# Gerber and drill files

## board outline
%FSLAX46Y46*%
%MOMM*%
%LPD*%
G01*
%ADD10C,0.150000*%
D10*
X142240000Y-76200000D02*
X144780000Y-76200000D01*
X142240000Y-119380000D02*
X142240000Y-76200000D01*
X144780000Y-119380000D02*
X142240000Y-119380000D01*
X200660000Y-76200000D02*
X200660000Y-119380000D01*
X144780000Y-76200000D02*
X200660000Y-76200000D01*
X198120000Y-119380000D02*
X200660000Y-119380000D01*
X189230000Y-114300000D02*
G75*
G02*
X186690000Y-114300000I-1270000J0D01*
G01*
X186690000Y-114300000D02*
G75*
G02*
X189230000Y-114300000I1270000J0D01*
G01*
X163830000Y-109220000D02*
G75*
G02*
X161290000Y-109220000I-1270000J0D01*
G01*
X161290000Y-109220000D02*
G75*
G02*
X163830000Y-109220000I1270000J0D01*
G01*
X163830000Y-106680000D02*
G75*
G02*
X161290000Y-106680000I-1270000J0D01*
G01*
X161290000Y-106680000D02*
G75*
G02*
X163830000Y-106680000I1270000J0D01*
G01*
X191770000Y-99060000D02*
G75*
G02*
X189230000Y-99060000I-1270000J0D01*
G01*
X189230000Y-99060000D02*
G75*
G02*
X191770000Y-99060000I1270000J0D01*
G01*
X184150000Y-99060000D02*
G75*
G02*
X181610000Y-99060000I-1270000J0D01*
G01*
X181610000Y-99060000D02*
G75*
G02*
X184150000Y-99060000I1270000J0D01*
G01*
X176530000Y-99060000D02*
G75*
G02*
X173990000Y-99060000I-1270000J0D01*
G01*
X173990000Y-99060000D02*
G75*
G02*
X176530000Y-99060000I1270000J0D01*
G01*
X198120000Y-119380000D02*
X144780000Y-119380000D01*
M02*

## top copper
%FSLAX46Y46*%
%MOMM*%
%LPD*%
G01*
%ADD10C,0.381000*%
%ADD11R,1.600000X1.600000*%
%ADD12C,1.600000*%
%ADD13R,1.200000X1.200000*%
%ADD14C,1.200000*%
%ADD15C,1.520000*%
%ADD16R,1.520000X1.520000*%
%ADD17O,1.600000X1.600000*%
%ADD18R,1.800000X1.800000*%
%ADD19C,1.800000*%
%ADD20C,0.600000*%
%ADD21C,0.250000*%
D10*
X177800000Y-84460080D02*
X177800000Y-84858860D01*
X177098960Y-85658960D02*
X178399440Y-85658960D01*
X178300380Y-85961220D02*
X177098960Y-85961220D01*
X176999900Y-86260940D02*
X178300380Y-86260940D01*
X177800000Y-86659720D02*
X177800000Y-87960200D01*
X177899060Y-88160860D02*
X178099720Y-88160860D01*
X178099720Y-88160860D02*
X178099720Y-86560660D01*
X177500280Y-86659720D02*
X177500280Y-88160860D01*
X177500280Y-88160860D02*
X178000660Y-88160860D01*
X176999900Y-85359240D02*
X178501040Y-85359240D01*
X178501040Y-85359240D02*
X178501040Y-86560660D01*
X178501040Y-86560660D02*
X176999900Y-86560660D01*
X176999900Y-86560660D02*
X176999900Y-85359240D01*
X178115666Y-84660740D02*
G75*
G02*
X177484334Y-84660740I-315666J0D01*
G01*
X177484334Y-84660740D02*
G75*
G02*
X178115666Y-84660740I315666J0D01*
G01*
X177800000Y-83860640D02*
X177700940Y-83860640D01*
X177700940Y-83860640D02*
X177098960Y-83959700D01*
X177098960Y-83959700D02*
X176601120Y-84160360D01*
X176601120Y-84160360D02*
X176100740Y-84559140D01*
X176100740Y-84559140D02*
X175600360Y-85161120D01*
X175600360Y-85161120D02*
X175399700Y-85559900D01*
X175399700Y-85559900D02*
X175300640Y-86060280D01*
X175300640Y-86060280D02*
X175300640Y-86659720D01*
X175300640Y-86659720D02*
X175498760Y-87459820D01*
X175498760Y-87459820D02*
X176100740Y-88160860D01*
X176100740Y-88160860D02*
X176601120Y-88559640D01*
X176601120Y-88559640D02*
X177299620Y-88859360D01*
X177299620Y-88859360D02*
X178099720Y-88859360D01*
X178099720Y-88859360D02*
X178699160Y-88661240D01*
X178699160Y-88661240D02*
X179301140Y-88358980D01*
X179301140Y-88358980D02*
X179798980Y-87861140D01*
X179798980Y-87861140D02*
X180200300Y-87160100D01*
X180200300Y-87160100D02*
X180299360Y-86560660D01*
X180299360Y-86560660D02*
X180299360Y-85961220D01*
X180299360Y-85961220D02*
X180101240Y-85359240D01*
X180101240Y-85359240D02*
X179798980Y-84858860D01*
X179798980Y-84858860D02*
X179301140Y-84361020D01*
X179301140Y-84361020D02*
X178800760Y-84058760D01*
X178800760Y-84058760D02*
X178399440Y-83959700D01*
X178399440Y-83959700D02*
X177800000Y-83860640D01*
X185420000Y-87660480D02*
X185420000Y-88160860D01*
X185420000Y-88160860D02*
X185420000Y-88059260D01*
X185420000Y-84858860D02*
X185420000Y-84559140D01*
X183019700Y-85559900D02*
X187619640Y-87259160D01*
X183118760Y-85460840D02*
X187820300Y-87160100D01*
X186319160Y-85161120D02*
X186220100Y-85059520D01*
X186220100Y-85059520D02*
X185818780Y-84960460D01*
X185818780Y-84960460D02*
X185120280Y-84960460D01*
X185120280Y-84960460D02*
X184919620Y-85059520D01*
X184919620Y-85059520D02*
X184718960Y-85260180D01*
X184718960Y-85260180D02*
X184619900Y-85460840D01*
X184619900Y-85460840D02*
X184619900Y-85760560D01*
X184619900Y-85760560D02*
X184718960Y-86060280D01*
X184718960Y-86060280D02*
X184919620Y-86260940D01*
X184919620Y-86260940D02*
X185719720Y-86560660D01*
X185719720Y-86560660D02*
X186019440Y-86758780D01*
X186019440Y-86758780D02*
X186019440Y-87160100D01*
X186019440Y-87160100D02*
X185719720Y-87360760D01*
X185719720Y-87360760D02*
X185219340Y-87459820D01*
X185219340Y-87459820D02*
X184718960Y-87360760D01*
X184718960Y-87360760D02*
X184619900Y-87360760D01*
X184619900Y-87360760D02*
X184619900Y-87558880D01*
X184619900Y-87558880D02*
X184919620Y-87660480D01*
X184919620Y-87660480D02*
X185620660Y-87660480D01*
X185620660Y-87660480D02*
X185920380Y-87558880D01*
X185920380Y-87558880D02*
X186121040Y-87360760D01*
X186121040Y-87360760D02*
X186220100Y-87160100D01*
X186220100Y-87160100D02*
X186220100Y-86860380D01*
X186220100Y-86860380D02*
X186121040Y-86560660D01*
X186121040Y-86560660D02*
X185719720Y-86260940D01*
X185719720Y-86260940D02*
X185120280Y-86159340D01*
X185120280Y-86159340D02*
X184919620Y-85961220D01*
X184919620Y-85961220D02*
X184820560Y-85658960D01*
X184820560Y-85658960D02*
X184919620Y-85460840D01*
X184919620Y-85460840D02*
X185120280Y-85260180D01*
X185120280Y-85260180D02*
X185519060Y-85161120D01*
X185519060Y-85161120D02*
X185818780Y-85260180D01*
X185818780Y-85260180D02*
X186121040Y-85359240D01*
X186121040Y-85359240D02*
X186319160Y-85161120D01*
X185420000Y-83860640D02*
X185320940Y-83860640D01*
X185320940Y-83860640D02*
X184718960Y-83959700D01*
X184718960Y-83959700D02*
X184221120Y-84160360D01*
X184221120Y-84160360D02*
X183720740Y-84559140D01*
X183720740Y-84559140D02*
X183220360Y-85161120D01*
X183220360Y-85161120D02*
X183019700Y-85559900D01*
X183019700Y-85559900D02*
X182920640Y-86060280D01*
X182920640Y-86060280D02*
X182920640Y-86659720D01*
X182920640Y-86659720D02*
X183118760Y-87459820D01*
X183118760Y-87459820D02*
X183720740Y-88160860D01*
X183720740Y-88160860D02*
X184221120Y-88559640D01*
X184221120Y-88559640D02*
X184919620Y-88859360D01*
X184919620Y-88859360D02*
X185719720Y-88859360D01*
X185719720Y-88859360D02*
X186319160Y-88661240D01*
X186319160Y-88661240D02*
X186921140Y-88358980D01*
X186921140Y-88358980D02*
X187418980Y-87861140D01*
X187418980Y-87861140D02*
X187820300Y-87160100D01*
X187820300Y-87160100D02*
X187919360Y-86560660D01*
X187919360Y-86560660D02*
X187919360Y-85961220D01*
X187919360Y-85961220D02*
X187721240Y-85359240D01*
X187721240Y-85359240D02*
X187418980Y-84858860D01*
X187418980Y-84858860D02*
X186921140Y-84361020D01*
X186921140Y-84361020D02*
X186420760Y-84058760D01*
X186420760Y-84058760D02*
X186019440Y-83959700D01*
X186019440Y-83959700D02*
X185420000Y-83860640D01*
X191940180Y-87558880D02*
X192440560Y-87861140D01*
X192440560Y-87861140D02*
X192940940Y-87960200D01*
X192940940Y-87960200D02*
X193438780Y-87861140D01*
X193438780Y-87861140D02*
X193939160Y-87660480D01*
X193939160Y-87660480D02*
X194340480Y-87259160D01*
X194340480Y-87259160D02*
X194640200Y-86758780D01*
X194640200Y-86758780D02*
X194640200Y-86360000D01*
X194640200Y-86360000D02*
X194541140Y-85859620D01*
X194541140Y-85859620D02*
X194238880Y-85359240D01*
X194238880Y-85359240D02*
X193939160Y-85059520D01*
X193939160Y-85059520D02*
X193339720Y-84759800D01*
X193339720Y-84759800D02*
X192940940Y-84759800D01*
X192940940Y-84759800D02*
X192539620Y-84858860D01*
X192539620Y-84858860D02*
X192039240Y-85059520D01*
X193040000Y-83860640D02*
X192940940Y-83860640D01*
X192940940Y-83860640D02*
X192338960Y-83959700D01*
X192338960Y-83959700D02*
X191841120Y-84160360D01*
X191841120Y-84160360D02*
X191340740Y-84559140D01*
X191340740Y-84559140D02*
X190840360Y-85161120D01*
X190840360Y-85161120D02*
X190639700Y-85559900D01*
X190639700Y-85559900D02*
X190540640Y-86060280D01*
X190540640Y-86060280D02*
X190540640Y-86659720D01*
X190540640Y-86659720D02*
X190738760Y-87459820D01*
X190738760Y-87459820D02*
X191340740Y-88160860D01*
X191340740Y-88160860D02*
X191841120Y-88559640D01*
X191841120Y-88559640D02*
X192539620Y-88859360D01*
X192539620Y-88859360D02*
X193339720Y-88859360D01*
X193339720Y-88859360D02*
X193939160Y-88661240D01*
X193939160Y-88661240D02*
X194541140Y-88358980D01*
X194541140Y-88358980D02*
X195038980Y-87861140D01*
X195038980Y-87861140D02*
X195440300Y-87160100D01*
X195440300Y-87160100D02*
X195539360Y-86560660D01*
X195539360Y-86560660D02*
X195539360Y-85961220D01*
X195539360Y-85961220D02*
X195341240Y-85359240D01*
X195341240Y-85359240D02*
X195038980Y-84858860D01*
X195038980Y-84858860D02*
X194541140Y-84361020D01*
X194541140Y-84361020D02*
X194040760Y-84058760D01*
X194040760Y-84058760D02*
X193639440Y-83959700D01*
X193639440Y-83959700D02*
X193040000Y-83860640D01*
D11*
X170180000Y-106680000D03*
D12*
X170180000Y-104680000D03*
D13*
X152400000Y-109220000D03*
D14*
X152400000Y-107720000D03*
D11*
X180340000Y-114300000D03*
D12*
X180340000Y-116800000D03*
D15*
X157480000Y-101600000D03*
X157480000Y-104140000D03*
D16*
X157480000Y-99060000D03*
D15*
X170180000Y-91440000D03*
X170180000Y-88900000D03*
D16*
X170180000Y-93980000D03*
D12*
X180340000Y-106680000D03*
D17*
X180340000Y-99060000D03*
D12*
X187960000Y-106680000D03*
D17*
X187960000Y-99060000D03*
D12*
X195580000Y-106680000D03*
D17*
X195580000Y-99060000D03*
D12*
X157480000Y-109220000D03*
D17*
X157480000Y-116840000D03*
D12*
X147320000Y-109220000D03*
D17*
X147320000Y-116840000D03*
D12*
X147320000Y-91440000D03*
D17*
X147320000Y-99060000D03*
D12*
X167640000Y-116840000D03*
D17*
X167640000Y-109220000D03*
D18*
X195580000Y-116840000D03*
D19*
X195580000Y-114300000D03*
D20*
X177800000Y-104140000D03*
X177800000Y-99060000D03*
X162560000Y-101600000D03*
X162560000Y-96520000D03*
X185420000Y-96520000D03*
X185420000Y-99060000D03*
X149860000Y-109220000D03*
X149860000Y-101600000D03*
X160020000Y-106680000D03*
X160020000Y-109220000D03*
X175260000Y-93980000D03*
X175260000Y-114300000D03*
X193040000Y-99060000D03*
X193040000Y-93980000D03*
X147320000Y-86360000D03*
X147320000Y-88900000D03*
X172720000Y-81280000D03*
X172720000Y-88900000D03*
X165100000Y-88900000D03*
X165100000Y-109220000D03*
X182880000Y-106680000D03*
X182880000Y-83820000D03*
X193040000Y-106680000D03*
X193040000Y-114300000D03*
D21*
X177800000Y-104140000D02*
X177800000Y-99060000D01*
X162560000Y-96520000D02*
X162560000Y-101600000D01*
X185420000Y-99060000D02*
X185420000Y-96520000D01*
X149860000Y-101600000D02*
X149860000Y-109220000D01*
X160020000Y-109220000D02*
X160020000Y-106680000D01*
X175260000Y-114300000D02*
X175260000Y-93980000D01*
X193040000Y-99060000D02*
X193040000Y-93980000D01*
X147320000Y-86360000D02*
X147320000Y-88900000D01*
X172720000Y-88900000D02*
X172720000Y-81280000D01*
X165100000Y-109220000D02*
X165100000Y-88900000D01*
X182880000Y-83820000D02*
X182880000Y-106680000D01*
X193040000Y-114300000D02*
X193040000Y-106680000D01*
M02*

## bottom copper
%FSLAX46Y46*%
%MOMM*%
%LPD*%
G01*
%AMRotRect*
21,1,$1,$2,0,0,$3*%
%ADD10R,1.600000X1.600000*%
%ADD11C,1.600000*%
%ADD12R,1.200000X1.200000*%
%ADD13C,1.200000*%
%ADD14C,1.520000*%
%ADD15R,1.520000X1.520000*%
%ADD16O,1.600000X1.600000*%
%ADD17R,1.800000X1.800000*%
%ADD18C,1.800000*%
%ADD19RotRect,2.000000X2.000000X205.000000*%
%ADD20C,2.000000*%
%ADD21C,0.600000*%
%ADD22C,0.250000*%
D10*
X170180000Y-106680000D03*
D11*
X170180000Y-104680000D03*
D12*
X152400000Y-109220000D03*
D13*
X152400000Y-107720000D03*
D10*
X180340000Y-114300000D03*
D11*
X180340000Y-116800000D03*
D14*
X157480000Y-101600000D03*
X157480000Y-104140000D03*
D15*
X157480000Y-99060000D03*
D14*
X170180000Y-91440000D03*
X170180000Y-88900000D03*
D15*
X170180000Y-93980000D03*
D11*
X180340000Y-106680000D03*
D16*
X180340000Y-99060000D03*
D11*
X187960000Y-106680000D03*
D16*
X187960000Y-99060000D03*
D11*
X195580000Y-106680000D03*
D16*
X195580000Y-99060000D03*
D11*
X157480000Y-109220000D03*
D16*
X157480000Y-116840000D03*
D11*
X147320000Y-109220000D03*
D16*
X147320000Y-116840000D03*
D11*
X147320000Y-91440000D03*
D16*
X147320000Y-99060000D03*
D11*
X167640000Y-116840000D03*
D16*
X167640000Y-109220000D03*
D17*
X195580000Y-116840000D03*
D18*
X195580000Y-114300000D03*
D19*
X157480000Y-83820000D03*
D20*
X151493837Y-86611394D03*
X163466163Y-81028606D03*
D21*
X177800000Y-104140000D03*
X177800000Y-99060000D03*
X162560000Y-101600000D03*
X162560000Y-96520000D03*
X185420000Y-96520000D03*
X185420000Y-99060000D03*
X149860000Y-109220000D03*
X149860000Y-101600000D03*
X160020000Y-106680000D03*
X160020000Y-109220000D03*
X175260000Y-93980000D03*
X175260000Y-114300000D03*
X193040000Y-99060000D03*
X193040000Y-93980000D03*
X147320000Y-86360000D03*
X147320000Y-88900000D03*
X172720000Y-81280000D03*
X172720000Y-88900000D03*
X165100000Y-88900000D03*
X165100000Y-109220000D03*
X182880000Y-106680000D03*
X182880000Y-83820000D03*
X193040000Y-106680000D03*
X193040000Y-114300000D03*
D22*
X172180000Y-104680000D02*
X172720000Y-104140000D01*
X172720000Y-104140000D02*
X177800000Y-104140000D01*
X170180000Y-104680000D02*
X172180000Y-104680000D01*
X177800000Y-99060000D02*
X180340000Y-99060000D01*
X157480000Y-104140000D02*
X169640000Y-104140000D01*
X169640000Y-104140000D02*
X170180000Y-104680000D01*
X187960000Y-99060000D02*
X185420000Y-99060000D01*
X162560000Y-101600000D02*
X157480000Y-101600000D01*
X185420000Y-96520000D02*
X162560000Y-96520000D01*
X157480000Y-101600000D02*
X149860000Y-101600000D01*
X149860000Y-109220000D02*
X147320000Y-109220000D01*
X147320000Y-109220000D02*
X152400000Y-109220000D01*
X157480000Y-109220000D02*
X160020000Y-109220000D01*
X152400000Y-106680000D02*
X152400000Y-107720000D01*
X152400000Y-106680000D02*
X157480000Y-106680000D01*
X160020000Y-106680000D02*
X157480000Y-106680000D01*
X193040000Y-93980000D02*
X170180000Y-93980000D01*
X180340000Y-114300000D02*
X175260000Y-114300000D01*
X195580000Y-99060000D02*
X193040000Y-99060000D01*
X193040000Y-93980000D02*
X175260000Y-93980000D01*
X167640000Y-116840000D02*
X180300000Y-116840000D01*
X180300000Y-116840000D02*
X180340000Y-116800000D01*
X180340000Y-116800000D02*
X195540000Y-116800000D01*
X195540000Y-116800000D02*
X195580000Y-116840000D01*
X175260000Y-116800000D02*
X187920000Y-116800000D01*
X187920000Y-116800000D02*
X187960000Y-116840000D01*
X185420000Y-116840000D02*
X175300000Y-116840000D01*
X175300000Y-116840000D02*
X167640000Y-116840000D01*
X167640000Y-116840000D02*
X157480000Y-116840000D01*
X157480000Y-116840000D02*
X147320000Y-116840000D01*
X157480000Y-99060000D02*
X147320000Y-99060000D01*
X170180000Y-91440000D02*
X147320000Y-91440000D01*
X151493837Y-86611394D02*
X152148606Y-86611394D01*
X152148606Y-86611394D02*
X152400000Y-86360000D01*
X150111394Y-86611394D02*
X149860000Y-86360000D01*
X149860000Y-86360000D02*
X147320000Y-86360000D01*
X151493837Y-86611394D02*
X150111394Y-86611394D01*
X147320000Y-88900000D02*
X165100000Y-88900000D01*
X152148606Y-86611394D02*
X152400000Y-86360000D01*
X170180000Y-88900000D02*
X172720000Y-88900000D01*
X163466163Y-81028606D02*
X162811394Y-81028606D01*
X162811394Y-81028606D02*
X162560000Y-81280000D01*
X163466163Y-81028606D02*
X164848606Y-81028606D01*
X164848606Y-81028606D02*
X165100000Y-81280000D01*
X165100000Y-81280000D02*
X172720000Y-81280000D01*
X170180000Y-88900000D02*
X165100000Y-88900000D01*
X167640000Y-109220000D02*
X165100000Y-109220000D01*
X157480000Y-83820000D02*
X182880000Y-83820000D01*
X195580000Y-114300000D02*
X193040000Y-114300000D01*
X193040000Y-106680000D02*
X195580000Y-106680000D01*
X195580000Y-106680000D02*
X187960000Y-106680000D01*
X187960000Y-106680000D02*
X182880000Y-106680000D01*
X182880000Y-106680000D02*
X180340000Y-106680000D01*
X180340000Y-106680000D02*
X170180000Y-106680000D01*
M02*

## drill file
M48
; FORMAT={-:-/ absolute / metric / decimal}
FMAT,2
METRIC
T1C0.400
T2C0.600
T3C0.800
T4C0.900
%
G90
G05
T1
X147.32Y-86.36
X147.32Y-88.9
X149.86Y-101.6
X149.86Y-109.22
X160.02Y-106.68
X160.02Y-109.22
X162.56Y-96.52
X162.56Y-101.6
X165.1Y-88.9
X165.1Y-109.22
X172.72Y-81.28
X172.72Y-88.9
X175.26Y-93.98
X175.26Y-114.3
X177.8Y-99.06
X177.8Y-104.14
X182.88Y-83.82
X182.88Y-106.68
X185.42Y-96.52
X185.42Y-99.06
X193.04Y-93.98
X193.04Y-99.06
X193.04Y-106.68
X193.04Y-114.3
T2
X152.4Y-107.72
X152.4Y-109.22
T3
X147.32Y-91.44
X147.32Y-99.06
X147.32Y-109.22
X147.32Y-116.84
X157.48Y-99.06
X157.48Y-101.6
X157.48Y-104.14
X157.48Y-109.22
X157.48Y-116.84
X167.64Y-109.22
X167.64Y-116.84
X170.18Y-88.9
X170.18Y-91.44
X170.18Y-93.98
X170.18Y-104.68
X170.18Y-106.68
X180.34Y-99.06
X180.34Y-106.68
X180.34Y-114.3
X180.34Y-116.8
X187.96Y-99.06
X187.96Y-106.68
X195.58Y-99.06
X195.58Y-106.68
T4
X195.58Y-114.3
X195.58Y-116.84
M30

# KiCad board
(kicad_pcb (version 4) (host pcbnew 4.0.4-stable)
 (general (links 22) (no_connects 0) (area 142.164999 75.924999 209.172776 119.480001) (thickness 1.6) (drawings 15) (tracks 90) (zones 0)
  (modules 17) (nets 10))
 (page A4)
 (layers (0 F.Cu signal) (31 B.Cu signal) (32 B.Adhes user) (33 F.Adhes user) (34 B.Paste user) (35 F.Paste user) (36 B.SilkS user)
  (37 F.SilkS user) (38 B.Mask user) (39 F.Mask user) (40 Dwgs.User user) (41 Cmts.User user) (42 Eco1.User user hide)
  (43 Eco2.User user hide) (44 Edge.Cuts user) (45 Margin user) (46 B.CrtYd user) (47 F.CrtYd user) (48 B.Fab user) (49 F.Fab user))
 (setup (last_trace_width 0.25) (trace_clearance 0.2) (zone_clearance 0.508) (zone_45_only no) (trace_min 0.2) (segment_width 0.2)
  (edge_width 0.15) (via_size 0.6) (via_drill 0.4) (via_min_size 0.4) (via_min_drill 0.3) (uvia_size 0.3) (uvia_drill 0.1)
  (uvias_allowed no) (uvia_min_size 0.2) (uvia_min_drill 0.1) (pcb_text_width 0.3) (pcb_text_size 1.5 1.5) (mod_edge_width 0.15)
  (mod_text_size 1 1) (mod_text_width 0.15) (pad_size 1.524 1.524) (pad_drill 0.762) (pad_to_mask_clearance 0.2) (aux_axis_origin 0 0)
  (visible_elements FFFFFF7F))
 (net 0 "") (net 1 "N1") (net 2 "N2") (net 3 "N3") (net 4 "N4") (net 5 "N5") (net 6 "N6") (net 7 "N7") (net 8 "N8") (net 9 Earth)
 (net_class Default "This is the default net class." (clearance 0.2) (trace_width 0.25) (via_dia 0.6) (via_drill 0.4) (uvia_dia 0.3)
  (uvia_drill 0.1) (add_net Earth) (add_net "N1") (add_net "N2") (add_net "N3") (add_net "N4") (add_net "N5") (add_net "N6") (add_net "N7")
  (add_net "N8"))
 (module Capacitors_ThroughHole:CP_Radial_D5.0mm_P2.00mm (layer F.Cu) (at 170.18 106.68 90)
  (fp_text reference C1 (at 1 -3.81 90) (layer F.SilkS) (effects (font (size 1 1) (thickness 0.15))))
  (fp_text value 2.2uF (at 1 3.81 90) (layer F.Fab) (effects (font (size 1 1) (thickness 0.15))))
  (pad 1 thru_hole rect (at 0 0 90) (size 1.6 1.6) (drill 0.8) (layers *.Cu *.Mask) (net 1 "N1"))
  (pad 2 thru_hole circle (at 2 0 90) (size 1.6 1.6) (drill 0.8) (layers *.Cu *.Mask) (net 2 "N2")))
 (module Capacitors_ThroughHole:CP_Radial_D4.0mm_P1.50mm (layer F.Cu) (at 152.4 109.22 90)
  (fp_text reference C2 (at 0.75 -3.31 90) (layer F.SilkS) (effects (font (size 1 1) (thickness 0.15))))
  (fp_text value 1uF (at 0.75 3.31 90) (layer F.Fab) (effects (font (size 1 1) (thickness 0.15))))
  (pad 1 thru_hole rect (at 0 0 90) (size 1.2 1.2) (drill 0.6) (layers *.Cu *.Mask) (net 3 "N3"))
  (pad 2 thru_hole circle (at 1.5 0 90) (size 1.2 1.2) (drill 0.6) (layers *.Cu *.Mask) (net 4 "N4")))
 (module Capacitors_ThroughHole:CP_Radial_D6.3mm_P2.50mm (layer F.Cu) (at 180.34 114.3 270)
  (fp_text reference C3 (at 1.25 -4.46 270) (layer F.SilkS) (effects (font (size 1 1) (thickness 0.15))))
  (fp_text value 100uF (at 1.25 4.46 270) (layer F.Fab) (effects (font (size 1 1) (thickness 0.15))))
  (pad 1 thru_hole rect (at 0 0 270) (size 1.6 1.6) (drill 0.8) (layers *.Cu *.Mask) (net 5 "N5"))
  (pad 2 thru_hole circle (at 2.5 0 270) (size 1.6 1.6) (drill 0.8) (layers *.Cu *.Mask) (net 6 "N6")))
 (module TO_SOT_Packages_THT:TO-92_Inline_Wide (layer F.Cu) (at 157.48 99.06 270)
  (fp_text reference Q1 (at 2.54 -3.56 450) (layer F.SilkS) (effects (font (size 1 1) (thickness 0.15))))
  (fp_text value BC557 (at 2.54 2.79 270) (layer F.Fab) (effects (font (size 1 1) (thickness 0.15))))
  (pad 2 thru_hole circle (at 2.54 0) (size 1.52 1.52) (drill 0.8) (layers *.Cu *.Mask) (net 3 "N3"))
  (pad 3 thru_hole circle (at 5.08 0) (size 1.52 1.52) (drill 0.8) (layers *.Cu *.Mask) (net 2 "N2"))
  (pad 1 thru_hole rect (at 0 0) (size 1.52 1.52) (drill 0.8) (layers *.Cu *.Mask) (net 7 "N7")))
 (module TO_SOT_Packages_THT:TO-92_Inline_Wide (layer F.Cu) (at 170.18 93.98 90)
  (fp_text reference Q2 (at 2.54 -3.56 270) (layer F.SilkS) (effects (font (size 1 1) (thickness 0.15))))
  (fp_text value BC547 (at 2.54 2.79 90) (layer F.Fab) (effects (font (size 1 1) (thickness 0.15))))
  (pad 2 thru_hole circle (at 2.54 0 180) (size 1.52 1.52) (drill 0.8) (layers *.Cu *.Mask) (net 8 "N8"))
  (pad 3 thru_hole circle (at 5.08 0 180) (size 1.52 1.52) (drill 0.8) (layers *.Cu *.Mask) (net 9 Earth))
  (pad 1 thru_hole rect (at 0 0 180) (size 1.52 1.52) (drill 0.8) (layers *.Cu *.Mask) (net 5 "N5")))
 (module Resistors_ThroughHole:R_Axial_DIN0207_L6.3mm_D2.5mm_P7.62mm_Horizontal (layer F.Cu) (at 180.34 106.68 90)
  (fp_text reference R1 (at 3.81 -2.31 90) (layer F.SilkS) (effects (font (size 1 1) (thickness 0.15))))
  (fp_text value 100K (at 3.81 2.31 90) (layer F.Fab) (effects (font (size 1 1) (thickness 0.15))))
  (pad 1 thru_hole circle (at 0 0 90) (size 1.6 1.6) (drill 0.8) (layers *.Cu *.Mask) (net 1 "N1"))
  (pad 2 thru_hole oval (at 7.62 0 90) (size 1.6 1.6) (drill 0.8) (layers *.Cu *.Mask) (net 2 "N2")))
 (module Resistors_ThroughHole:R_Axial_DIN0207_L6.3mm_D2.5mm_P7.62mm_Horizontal (layer F.Cu) (at 187.96 106.68 90)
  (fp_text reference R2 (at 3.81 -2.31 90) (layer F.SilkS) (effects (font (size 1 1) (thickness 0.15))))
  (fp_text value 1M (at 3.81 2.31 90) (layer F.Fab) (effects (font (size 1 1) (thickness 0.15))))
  (pad 1 thru_hole circle (at 0 0 90) (size 1.6 1.6) (drill 0.8) (layers *.Cu *.Mask) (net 1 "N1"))
  (pad 2 thru_hole oval (at 7.62 0 90) (size 1.6 1.6) (drill 0.8) (layers *.Cu *.Mask) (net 3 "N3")))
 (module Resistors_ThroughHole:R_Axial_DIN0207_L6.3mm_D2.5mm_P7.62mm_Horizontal (layer F.Cu) (at 195.58 106.68 90)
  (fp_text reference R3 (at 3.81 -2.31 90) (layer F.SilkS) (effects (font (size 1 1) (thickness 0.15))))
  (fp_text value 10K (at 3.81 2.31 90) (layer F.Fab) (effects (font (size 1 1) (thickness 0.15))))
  (pad 1 thru_hole circle (at 0 0 90) (size 1.6 1.6) (drill 0.8) (layers *.Cu *.Mask) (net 1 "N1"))
  (pad 2 thru_hole oval (at 7.62 0 90) (size 1.6 1.6) (drill 0.8) (layers *.Cu *.Mask) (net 5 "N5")))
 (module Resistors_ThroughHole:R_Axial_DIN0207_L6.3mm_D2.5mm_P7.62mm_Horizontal (layer F.Cu) (at 157.48 109.22 270)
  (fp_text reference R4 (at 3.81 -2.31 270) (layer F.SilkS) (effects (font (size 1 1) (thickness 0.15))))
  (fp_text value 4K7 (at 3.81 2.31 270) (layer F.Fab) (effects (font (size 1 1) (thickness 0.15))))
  (pad 1 thru_hole circle (at 0 0 270) (size 1.6 1.6) (drill 0.8) (layers *.Cu *.Mask) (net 4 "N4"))
  (pad 2 thru_hole oval (at 7.62 0 270) (size 1.6 1.6) (drill 0.8) (layers *.Cu *.Mask) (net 6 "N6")))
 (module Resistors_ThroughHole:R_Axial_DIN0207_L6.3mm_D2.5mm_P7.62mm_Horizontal (layer F.Cu) (at 147.32 109.22 270)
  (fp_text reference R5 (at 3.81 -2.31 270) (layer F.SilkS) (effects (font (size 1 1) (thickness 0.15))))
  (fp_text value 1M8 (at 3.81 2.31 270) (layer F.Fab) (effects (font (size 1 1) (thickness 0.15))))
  (pad 1 thru_hole circle (at 0 0 270) (size 1.6 1.6) (drill 0.8) (layers *.Cu *.Mask) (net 3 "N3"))
  (pad 2 thru_hole oval (at 7.62 0 270) (size 1.6 1.6) (drill 0.8) (layers *.Cu *.Mask) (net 6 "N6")))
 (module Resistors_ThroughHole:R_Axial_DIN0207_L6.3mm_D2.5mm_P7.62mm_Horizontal (layer F.Cu) (at 147.32 91.44 270)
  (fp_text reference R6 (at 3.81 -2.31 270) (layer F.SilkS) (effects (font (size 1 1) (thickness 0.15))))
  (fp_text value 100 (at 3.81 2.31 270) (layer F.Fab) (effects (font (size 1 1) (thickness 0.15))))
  (pad 1 thru_hole circle (at 0 0 270) (size 1.6 1.6) (drill 0.8) (layers *.Cu *.Mask) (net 8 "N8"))
  (pad 2 thru_hole oval (at 7.62 0 270) (size 1.6 1.6) (drill 0.8) (layers *.Cu *.Mask) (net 7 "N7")))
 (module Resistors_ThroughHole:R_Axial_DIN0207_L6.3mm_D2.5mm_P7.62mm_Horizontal (layer F.Cu) (at 167.64 116.84 90)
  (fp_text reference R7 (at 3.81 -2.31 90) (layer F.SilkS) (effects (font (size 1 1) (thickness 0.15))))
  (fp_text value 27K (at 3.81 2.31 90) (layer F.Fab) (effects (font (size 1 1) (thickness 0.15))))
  (pad 1 thru_hole circle (at 0 0 90) (size 1.6 1.6) (drill 0.8) (layers *.Cu *.Mask) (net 6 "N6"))
  (pad 2 thru_hole oval (at 7.62 0 90) (size 1.6 1.6) (drill 0.8) (layers *.Cu *.Mask) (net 9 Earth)))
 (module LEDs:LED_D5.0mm (layer F.Cu) (at 195.58 116.84 90)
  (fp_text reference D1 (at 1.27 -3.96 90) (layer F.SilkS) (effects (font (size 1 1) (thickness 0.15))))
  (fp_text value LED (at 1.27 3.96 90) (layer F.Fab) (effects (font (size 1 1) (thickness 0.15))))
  (pad 1 thru_hole rect (at 0 0 90) (size 1.8 1.8) (drill 0.9) (layers *.Cu *.Mask) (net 6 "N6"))
  (pad 2 thru_hole circle (at 2.54 0 90) (size 1.8 1.8) (drill 0.9) (layers *.Cu *.Mask) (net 1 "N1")))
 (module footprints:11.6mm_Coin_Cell (layer F.Cu) (at 157.48 83.82 205) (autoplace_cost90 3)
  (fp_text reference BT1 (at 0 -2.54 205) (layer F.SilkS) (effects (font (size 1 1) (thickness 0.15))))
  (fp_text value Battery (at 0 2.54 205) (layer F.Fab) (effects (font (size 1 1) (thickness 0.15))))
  (pad 1 smd rect (at 0 0 205) (size 2 2) (layers B.Cu F.Paste F.Mask) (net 1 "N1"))
  (pad 2 smd circle (at 6.605 0 205) (size 2 2) (layers B.Cu F.Paste F.Mask) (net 9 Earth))
  (pad 2 smd circle (at -6.605 0 205) (size 2 2) (layers B.Cu F.Paste F.Mask) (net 9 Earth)))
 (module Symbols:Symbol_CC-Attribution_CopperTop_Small (layer F.Cu) (at 177.8 86.36)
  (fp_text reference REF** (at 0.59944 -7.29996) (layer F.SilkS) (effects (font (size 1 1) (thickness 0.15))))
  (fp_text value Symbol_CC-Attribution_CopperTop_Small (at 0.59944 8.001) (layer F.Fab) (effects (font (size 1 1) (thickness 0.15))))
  (fp_line (start 0 -1.89992) (end 0 -1.50114) (layer F.Cu) (width 0.381))
  (fp_line (start -0.70104 -0.70104) (end 0.59944 -0.70104) (layer F.Cu) (width 0.381))
  (fp_line (start 0.50038 -0.39878) (end -0.70104 -0.39878) (layer F.Cu) (width 0.381))
  (fp_line (start -0.8001 -0.09906) (end 0.50038 -0.09906) (layer F.Cu) (width 0.381))
  (fp_line (start 0 0.29972) (end 0 1.6002) (layer F.Cu) (width 0.381))
  (fp_line (start 0.09906 1.80086) (end 0.29972 1.80086) (layer F.Cu) (width 0.381))
  (fp_line (start 0.29972 1.80086) (end 0.29972 0.20066) (layer F.Cu) (width 0.381))
  (fp_line (start -0.29972 0.29972) (end -0.29972 1.80086) (layer F.Cu) (width 0.381))
  (fp_line (start -0.29972 1.80086) (end 0.20066 1.80086) (layer F.Cu) (width 0.381))
  (fp_line (start -0.8001 -1.00076) (end 0.70104 -1.00076) (layer F.Cu) (width 0.381))
  (fp_line (start 0.70104 -1.00076) (end 0.70104 0.20066) (layer F.Cu) (width 0.381))
  (fp_line (start 0.70104 0.20066) (end -0.8001 0.20066) (layer F.Cu) (width 0.381))
  (fp_line (start -0.8001 0.20066) (end -0.8001 -1.00076) (layer F.Cu) (width 0.381))
  (fp_circle (center 0 -1.69926) (end 0.09906 -1.39954) (layer F.Cu) (width 0.381))
  (fp_line (start 0 -2.49936) (end -0.09906 -2.49936) (layer F.Cu) (width 0.381))
  (fp_line (start -0.09906 -2.49936) (end -0.70104 -2.4003) (layer F.Cu) (width 0.381))
  (fp_line (start -0.70104 -2.4003) (end -1.19888 -2.19964) (layer F.Cu) (width 0.381))
  (fp_line (start -1.19888 -2.19964) (end -1.69926 -1.80086) (layer F.Cu) (width 0.381))
  (fp_line (start -1.69926 -1.80086) (end -2.19964 -1.19888) (layer F.Cu) (width 0.381))
  (fp_line (start -2.19964 -1.19888) (end -2.4003 -0.8001) (layer F.Cu) (width 0.381))
  (fp_line (start -2.4003 -0.8001) (end -2.49936 -0.29972) (layer F.Cu) (width 0.381))
  (fp_line (start -2.49936 -0.29972) (end -2.49936 0.29972) (layer F.Cu) (width 0.381))
  (fp_line (start -2.49936 0.29972) (end -2.30124 1.09982) (layer F.Cu) (width 0.381))
  (fp_line (start -2.30124 1.09982) (end -1.69926 1.80086) (layer F.Cu) (width 0.381))
  (fp_line (start -1.69926 1.80086) (end -1.19888 2.19964) (layer F.Cu) (width 0.381))
  (fp_line (start -1.19888 2.19964) (end -0.50038 2.49936) (layer F.Cu) (width 0.381))
  (fp_line (start -0.50038 2.49936) (end 0.29972 2.49936) (layer F.Cu) (width 0.381))
  (fp_line (start 0.29972 2.49936) (end 0.89916 2.30124) (layer F.Cu) (width 0.381))
  (fp_line (start 0.89916 2.30124) (end 1.50114 1.99898) (layer F.Cu) (width 0.381))
  (fp_line (start 1.50114 1.99898) (end 1.99898 1.50114) (layer F.Cu) (width 0.381))
  (fp_line (start 1.99898 1.50114) (end 2.4003 0.8001) (layer F.Cu) (width 0.381))
  (fp_line (start 2.4003 0.8001) (end 2.49936 0.20066) (layer F.Cu) (width 0.381))
  (fp_line (start 2.49936 0.20066) (end 2.49936 -0.39878) (layer F.Cu) (width 0.381))
  (fp_line (start 2.49936 -0.39878) (end 2.30124 -1.00076) (layer F.Cu) (width 0.381))
  (fp_line (start 2.30124 -1.00076) (end 1.99898 -1.50114) (layer F.Cu) (width 0.381))
  (fp_line (start 1.99898 -1.50114) (end 1.50114 -1.99898) (layer F.Cu) (width 0.381))
  (fp_line (start 1.50114 -1.99898) (end 1.00076 -2.30124) (layer F.Cu) (width 0.381))
  (fp_line (start 1.00076 -2.30124) (end 0.59944 -2.4003) (layer F.Cu) (width 0.381))
  (fp_line (start 0.59944 -2.4003) (end 0 -2.49936) (layer F.Cu) (width 0.381)))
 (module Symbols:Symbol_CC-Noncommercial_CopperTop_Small (layer F.Cu) (at 185.42 86.36)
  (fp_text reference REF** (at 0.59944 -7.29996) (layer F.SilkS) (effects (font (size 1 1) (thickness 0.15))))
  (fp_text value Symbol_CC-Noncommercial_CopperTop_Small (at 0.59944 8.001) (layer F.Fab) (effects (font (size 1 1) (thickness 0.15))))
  (fp_line (start 0 1.30048) (end 0 1.80086) (layer F.Cu) (width 0.381))
  (fp_line (start 0 1.80086) (end 0 1.69926) (layer F.Cu) (width 0.381))
  (fp_line (start 0 -1.50114) (end 0 -1.80086) (layer F.Cu) (width 0.381))
  (fp_line (start -2.4003 -0.8001) (end 2.19964 0.89916) (layer F.Cu) (width 0.381))
  (fp_line (start -2.30124 -0.89916) (end 2.4003 0.8001) (layer F.Cu) (width 0.381))
  (fp_line (start 0.89916 -1.19888) (end 0.8001 -1.30048) (layer F.Cu) (width 0.381))
  (fp_line (start 0.8001 -1.30048) (end 0.39878 -1.39954) (layer F.Cu) (width 0.381))
  (fp_line (start 0.39878 -1.39954) (end -0.29972 -1.39954) (layer F.Cu) (width 0.381))
  (fp_line (start -0.29972 -1.39954) (end -0.50038 -1.30048) (layer F.Cu) (width 0.381))
  (fp_line (start -0.50038 -1.30048) (end -0.70104 -1.09982) (layer F.Cu) (width 0.381))
  (fp_line (start -0.70104 -1.09982) (end -0.8001 -0.89916) (layer F.Cu) (width 0.381))
  (fp_line (start -0.8001 -0.89916) (end -0.8001 -0.59944) (layer F.Cu) (width 0.381))
  (fp_line (start -0.8001 -0.59944) (end -0.70104 -0.29972) (layer F.Cu) (width 0.381))
  (fp_line (start -0.70104 -0.29972) (end -0.50038 -0.09906) (layer F.Cu) (width 0.381))
  (fp_line (start -0.50038 -0.09906) (end 0.29972 0.20066) (layer F.Cu) (width 0.381))
  (fp_line (start 0.29972 0.20066) (end 0.59944 0.39878) (layer F.Cu) (width 0.381))
  (fp_line (start 0.59944 0.39878) (end 0.59944 0.8001) (layer F.Cu) (width 0.381))
  (fp_line (start 0.59944 0.8001) (end 0.29972 1.00076) (layer F.Cu) (width 0.381))
  (fp_line (start 0.29972 1.00076) (end -0.20066 1.09982) (layer F.Cu) (width 0.381))
  (fp_line (start -0.20066 1.09982) (end -0.70104 1.00076) (layer F.Cu) (width 0.381))
  (fp_line (start -0.70104 1.00076) (end -0.8001 1.00076) (layer F.Cu) (width 0.381))
  (fp_line (start -0.8001 1.00076) (end -0.8001 1.19888) (layer F.Cu) (width 0.381))
  (fp_line (start -0.8001 1.19888) (end -0.50038 1.30048) (layer F.Cu) (width 0.381))
  (fp_line (start -0.50038 1.30048) (end 0.20066 1.30048) (layer F.Cu) (width 0.381))
  (fp_line (start 0.20066 1.30048) (end 0.50038 1.19888) (layer F.Cu) (width 0.381))
  (fp_line (start 0.50038 1.19888) (end 0.70104 1.00076) (layer F.Cu) (width 0.381))
  (fp_line (start 0.70104 1.00076) (end 0.8001 0.8001) (layer F.Cu) (width 0.381))
  (fp_line (start 0.8001 0.8001) (end 0.8001 0.50038) (layer F.Cu) (width 0.381))
  (fp_line (start 0.8001 0.50038) (end 0.70104 0.20066) (layer F.Cu) (width 0.381))
  (fp_line (start 0.70104 0.20066) (end 0.29972 -0.09906) (layer F.Cu) (width 0.381))
  (fp_line (start 0.29972 -0.09906) (end -0.29972 -0.20066) (layer F.Cu) (width 0.381))
  (fp_line (start -0.29972 -0.20066) (end -0.50038 -0.39878) (layer F.Cu) (width 0.381))
  (fp_line (start -0.50038 -0.39878) (end -0.59944 -0.70104) (layer F.Cu) (width 0.381))
  (fp_line (start -0.59944 -0.70104) (end -0.50038 -0.89916) (layer F.Cu) (width 0.381))
  (fp_line (start -0.50038 -0.89916) (end -0.29972 -1.09982) (layer F.Cu) (width 0.381))
  (fp_line (start -0.29972 -1.09982) (end 0.09906 -1.19888) (layer F.Cu) (width 0.381))
  (fp_line (start 0.09906 -1.19888) (end 0.39878 -1.09982) (layer F.Cu) (width 0.381))
  (fp_line (start 0.39878 -1.09982) (end 0.70104 -1.00076) (layer F.Cu) (width 0.381))
  (fp_line (start 0.70104 -1.00076) (end 0.89916 -1.19888) (layer F.Cu) (width 0.381))
  (fp_line (start 0 -2.49936) (end -0.09906 -2.49936) (layer F.Cu) (width 0.381))
  (fp_line (start -0.09906 -2.49936) (end -0.70104 -2.4003) (layer F.Cu) (width 0.381))
  (fp_line (start -0.70104 -2.4003) (end -1.19888 -2.19964) (layer F.Cu) (width 0.381))
  (fp_line (start -1.19888 -2.19964) (end -1.69926 -1.80086) (layer F.Cu) (width 0.381))
  (fp_line (start -1.69926 -1.80086) (end -2.19964 -1.19888) (layer F.Cu) (width 0.381))
  (fp_line (start -2.19964 -1.19888) (end -2.4003 -0.8001) (layer F.Cu) (width 0.381))
  (fp_line (start -2.4003 -0.8001) (end -2.49936 -0.29972) (layer F.Cu) (width 0.381))
  (fp_line (start -2.49936 -0.29972) (end -2.49936 0.29972) (layer F.Cu) (width 0.381))
  (fp_line (start -2.49936 0.29972) (end -2.30124 1.09982) (layer F.Cu) (width 0.381))
  (fp_line (start -2.30124 1.09982) (end -1.69926 1.80086) (layer F.Cu) (width 0.381))
  (fp_line (start -1.69926 1.80086) (end -1.19888 2.19964) (layer F.Cu) (width 0.381))
  (fp_line (start -1.19888 2.19964) (end -0.50038 2.49936) (layer F.Cu) (width 0.381))
  (fp_line (start -0.50038 2.49936) (end 0.29972 2.49936) (layer F.Cu) (width 0.381))
  (fp_line (start 0.29972 2.49936) (end 0.89916 2.30124) (layer F.Cu) (width 0.381))
  (fp_line (start 0.89916 2.30124) (end 1.50114 1.99898) (layer F.Cu) (width 0.381))
  (fp_line (start 1.50114 1.99898) (end 1.99898 1.50114) (layer F.Cu) (width 0.381))
  (fp_line (start 1.99898 1.50114) (end 2.4003 0.8001) (layer F.Cu) (width 0.381))
  (fp_line (start 2.4003 0.8001) (end 2.49936 0.20066) (layer F.Cu) (width 0.381))
  (fp_line (start 2.49936 0.20066) (end 2.49936 -0.39878) (layer F.Cu) (width 0.381))
  (fp_line (start 2.49936 -0.39878) (end 2.30124 -1.00076) (layer F.Cu) (width 0.381))
  (fp_line (start 2.30124 -1.00076) (end 1.99898 -1.50114) (layer F.Cu) (width 0.381))
  (fp_line (start 1.99898 -1.50114) (end 1.50114 -1.99898) (layer F.Cu) (width 0.381))
  (fp_line (start 1.50114 -1.99898) (end 1.00076 -2.30124) (layer F.Cu) (width 0.381))
  (fp_line (start 1.00076 -2.30124) (end 0.59944 -2.4003) (layer F.Cu) (width 0.381))
  (fp_line (start 0.59944 -2.4003) (end 0 -2.49936) (layer F.Cu) (width 0.381)))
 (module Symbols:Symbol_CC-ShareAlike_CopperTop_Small (layer F.Cu) (at 193.04 86.36)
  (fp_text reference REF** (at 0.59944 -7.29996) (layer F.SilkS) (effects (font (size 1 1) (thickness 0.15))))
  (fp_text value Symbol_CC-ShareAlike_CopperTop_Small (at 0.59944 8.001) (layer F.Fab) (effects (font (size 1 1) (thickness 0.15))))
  (fp_line (start -1.09982 1.19888) (end -0.59944 1.50114) (layer F.Cu) (width 0.381))
  (fp_line (start -0.59944 1.50114) (end -0.09906 1.6002) (layer F.Cu) (width 0.381))
  (fp_line (start -0.09906 1.6002) (end 0.39878 1.50114) (layer F.Cu) (width 0.381))
  (fp_line (start 0.39878 1.50114) (end 0.89916 1.30048) (layer F.Cu) (width 0.381))
  (fp_line (start 0.89916 1.30048) (end 1.30048 0.89916) (layer F.Cu) (width 0.381))
  (fp_line (start 1.30048 0.89916) (end 1.6002 0.39878) (layer F.Cu) (width 0.381))
  (fp_line (start 1.6002 0.39878) (end 1.6002 0) (layer F.Cu) (width 0.381))
  (fp_line (start 1.6002 0) (end 1.50114 -0.50038) (layer F.Cu) (width 0.381))
  (fp_line (start 1.50114 -0.50038) (end 1.19888 -1.00076) (layer F.Cu) (width 0.381))
  (fp_line (start 1.19888 -1.00076) (end 0.89916 -1.30048) (layer F.Cu) (width 0.381))
  (fp_line (start 0.89916 -1.30048) (end 0.29972 -1.6002) (layer F.Cu) (width 0.381))
  (fp_line (start 0.29972 -1.6002) (end -0.09906 -1.6002) (layer F.Cu) (width 0.381))
  (fp_line (start -0.09906 -1.6002) (end -0.50038 -1.50114) (layer F.Cu) (width 0.381))
  (fp_line (start -0.50038 -1.50114) (end -1.00076 -1.30048) (layer F.Cu) (width 0.381))
  (fp_line (start 0 -2.49936) (end -0.09906 -2.49936) (layer F.Cu) (width 0.381))
  (fp_line (start -0.09906 -2.49936) (end -0.70104 -2.4003) (layer F.Cu) (width 0.381))
  (fp_line (start -0.70104 -2.4003) (end -1.19888 -2.19964) (layer F.Cu) (width 0.381))
  (fp_line (start -1.19888 -2.19964) (end -1.69926 -1.80086) (layer F.Cu) (width 0.381))
  (fp_line (start -1.69926 -1.80086) (end -2.19964 -1.19888) (layer F.Cu) (width 0.381))
  (fp_line (start -2.19964 -1.19888) (end -2.4003 -0.8001) (layer F.Cu) (width 0.381))
  (fp_line (start -2.4003 -0.8001) (end -2.49936 -0.29972) (layer F.Cu) (width 0.381))
  (fp_line (start -2.49936 -0.29972) (end -2.49936 0.29972) (layer F.Cu) (width 0.381))
  (fp_line (start -2.49936 0.29972) (end -2.30124 1.09982) (layer F.Cu) (width 0.381))
  (fp_line (start -2.30124 1.09982) (end -1.69926 1.80086) (layer F.Cu) (width 0.381))
  (fp_line (start -1.69926 1.80086) (end -1.19888 2.19964) (layer F.Cu) (width 0.381))
  (fp_line (start -1.19888 2.19964) (end -0.50038 2.49936) (layer F.Cu) (width 0.381))
  (fp_line (start -0.50038 2.49936) (end 0.29972 2.49936) (layer F.Cu) (width 0.381))
  (fp_line (start 0.29972 2.49936) (end 0.89916 2.30124) (layer F.Cu) (width 0.381))
  (fp_line (start 0.89916 2.30124) (end 1.50114 1.99898) (layer F.Cu) (width 0.381))
  (fp_line (start 1.50114 1.99898) (end 1.99898 1.50114) (layer F.Cu) (width 0.381))
  (fp_line (start 1.99898 1.50114) (end 2.4003 0.8001) (layer F.Cu) (width 0.381))
  (fp_line (start 2.4003 0.8001) (end 2.49936 0.20066) (layer F.Cu) (width 0.381))
  (fp_line (start 2.49936 0.20066) (end 2.49936 -0.39878) (layer F.Cu) (width 0.381))
  (fp_line (start 2.49936 -0.39878) (end 2.30124 -1.00076) (layer F.Cu) (width 0.381))
  (fp_line (start 2.30124 -1.00076) (end 1.99898 -1.50114) (layer F.Cu) (width 0.381))
  (fp_line (start 1.99898 -1.50114) (end 1.50114 -1.99898) (layer F.Cu) (width 0.381))
  (fp_line (start 1.50114 -1.99898) (end 1.00076 -2.30124) (layer F.Cu) (width 0.381))
  (fp_line (start 1.00076 -2.30124) (end 0.59944 -2.4003) (layer F.Cu) (width 0.381))
  (fp_line (start 0.59944 -2.4003) (end 0 -2.49936) (layer F.Cu) (width 0.381)))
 (gr_line (start 142.24 76.2) (end 144.78 76.2) (angle 90) (layer Edge.Cuts) (width 0.15))
 (gr_line (start 142.24 119.38) (end 142.24 76.2) (angle 90) (layer Edge.Cuts) (width 0.15))
 (gr_line (start 144.78 119.38) (end 142.24 119.38) (angle 90) (layer Edge.Cuts) (width 0.15))
 (gr_line (start 200.66 76.2) (end 200.66 119.38) (angle 90) (layer Edge.Cuts) (width 0.15))
 (gr_line (start 144.78 76.2) (end 200.66 76.2) (angle 90) (layer Edge.Cuts) (width 0.15))
 (gr_line (start 198.12 119.38) (end 200.66 119.38) (angle 90) (layer Edge.Cuts) (width 0.15))
 (gr_circle (center 187.96 114.3) (end 189.23 114.3) (layer Edge.Cuts) (width 0.15))
 (gr_circle (center 162.56 109.22) (end 163.83 109.22) (layer Edge.Cuts) (width 0.15))
 (gr_circle (center 162.56 106.68) (end 163.83 106.68) (layer Edge.Cuts) (width 0.15))
 (gr_circle (center 190.5 99.06) (end 191.77 99.06) (layer Edge.Cuts) (width 0.15))
 (gr_circle (center 182.88 99.06) (end 184.15 99.06) (layer Edge.Cuts) (width 0.15))
 (gr_circle (center 175.26 99.06) (end 176.53 99.06) (layer Edge.Cuts) (width 0.15))
 (gr_line (start 198.12 119.38) (end 144.78 119.38) (angle 90) (layer Edge.Cuts) (width 0.15))
 (via (at 177.8 104.14) (size 0.6) (drill 0.4) (layers F.Cu B.Cu) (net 2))
 (segment (start 172.18 104.68) (end 172.72 104.14) (width 0.25) (layer B.Cu) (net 2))
 (segment (start 172.72 104.14) (end 177.8 104.14) (width 0.25) (layer B.Cu) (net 2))
 (segment (start 170.18 104.68) (end 172.18 104.68) (width 0.25) (layer B.Cu) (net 2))
 (segment (start 177.8 99.06) (end 180.34 99.06) (width 0.25) (layer B.Cu) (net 2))
 (via (at 177.8 99.06) (size 0.6) (drill 0.4) (layers F.Cu B.Cu) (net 2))
 (segment (start 177.8 104.14) (end 177.8 99.06) (width 0.25) (layer F.Cu) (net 2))
 (segment (start 157.48 104.14) (end 169.64 104.14) (width 0.25) (layer B.Cu) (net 2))
 (segment (start 169.64 104.14) (end 170.18 104.68) (width 0.25) (layer B.Cu) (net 2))
 (segment (start 187.96 99.06) (end 185.42 99.06) (width 0.25) (layer B.Cu) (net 3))
 (segment (start 162.56 101.6) (end 157.48 101.6) (width 0.25) (layer B.Cu) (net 3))
 (via (at 162.56 101.6) (size 0.6) (drill 0.4) (layers F.Cu B.Cu) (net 3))
 (segment (start 162.56 96.52) (end 162.56 101.6) (width 0.25) (layer F.Cu) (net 3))
 (via (at 162.56 96.52) (size 0.6) (drill 0.4) (layers F.Cu B.Cu) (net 3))
 (segment (start 185.42 96.52) (end 162.56 96.52) (width 0.25) (layer B.Cu) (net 3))
 (via (at 185.42 96.52) (size 0.6) (drill 0.4) (layers F.Cu B.Cu) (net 3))
 (segment (start 185.42 99.06) (end 185.42 96.52) (width 0.25) (layer F.Cu) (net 3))
 (via (at 185.42 99.06) (size 0.6) (drill 0.4) (layers F.Cu B.Cu) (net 3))
 (segment (start 157.48 101.6) (end 149.86 101.6) (width 0.25) (layer B.Cu) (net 3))
 (segment (start 149.86 109.22) (end 147.32 109.22) (width 0.25) (layer B.Cu) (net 3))
 (via (at 149.86 109.22) (size 0.6) (drill 0.4) (layers F.Cu B.Cu) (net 3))
 (segment (start 149.86 101.6) (end 149.86 109.22) (width 0.25) (layer F.Cu) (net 3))
 (via (at 149.86 101.6) (size 0.6) (drill 0.4) (layers F.Cu B.Cu) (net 3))
 (segment (start 147.32 109.22) (end 152.4 109.22) (width 0.25) (layer B.Cu) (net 3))
 (segment (start 157.48 109.22) (end 160.02 109.22) (width 0.25) (layer B.Cu) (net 4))
 (segment (start 152.4 106.68) (end 152.4 107.72) (width 0.25) (layer B.Cu) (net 4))
 (segment (start 152.4 106.68) (end 157.48 106.68) (width 0.25) (layer B.Cu) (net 4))
 (segment (start 160.02 106.68) (end 157.48 106.68) (width 0.25) (layer B.Cu) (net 4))
 (via (at 160.02 106.68) (size 0.6) (drill 0.4) (layers F.Cu B.Cu) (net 4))
 (segment (start 160.02 109.22) (end 160.02 106.68) (width 0.25) (layer F.Cu) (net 4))
 (via (at 160.02 109.22) (size 0.6) (drill 0.4) (layers F.Cu B.Cu) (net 4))
 (segment (start 193.04 93.98) (end 170.18 93.98) (width 0.25) (layer B.Cu) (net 5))
 (via (at 175.26 93.98) (size 0.6) (drill 0.4) (layers F.Cu B.Cu) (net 5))
 (segment (start 180.34 114.3) (end 175.26 114.3) (width 0.25) (layer B.Cu) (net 5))
 (via (at 175.26 114.3) (size 0.6) (drill 0.4) (layers F.Cu B.Cu) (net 5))
 (segment (start 175.26 114.3) (end 175.26 93.98) (width 0.25) (layer F.Cu) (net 5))
 (segment (start 195.58 99.06) (end 193.04 99.06) (width 0.25) (layer B.Cu) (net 5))
 (via (at 193.04 99.06) (size 0.6) (drill 0.4) (layers F.Cu B.Cu) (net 5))
 (segment (start 193.04 93.98) (end 175.26 93.98) (width 0.25) (layer B.Cu) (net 5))
 (via (at 193.04 93.98) (size 0.6) (drill 0.4) (layers F.Cu B.Cu) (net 5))
 (segment (start 193.04 99.06) (end 193.04 93.98) (width 0.25) (layer F.Cu) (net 5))
 (segment (start 167.64 116.84) (end 180.3 116.84) (width 0.25) (layer B.Cu) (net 6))
 (segment (start 180.3 116.84) (end 180.34 116.8) (width 0.25) (layer B.Cu) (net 6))
 (segment (start 180.34 116.8) (end 195.54 116.8) (width 0.25) (layer B.Cu) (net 6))
 (segment (start 195.54 116.8) (end 195.58 116.84) (width 0.25) (layer B.Cu) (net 6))
 (segment (start 175.26 116.8) (end 187.92 116.8) (width 0.25) (layer B.Cu) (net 6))
 (segment (start 187.92 116.8) (end 187.96 116.84) (width 0.25) (layer B.Cu) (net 6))
 (segment (start 185.42 116.84) (end 175.3 116.84) (width 0.25) (layer B.Cu) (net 6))
 (segment (start 175.3 116.84) (end 167.64 116.84) (width 0.25) (layer B.Cu) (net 6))
 (segment (start 167.64 116.84) (end 157.48 116.84) (width 0.25) (layer B.Cu) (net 6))
 (segment (start 157.48 116.84) (end 147.32 116.84) (width 0.25) (layer B.Cu) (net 6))
 (segment (start 157.48 99.06) (end 147.32 99.06) (width 0.25) (layer B.Cu) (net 7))
 (segment (start 170.18 91.44) (end 147.32 91.44) (width 0.25) (layer B.Cu) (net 8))
 (segment (start 151.493837 86.611394) (end 152.148606 86.611394) (width 0.25) (layer B.Cu) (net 9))
 (segment (start 152.148606 86.611394) (end 152.4 86.36) (width 0.25) (layer B.Cu) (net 9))
 (via (at 147.32 86.36) (size 0.6) (drill 0.4) (layers F.Cu B.Cu) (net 9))
 (segment (start 150.111394 86.611394) (end 149.86 86.36) (width 0.25) (layer B.Cu) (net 9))
 (segment (start 149.86 86.36) (end 147.32 86.36) (width 0.25) (layer B.Cu) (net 9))
 (segment (start 151.493837 86.611394) (end 150.111394 86.611394) (width 0.25) (layer B.Cu) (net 9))
 (segment (start 147.32 88.9) (end 165.1 88.9) (width 0.25) (layer B.Cu) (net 9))
 (via (at 147.32 88.9) (size 0.6) (drill 0.4) (layers F.Cu B.Cu) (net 9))
 (segment (start 147.32 86.36) (end 147.32 88.9) (width 0.25) (layer F.Cu) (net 9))
 (segment (start 152.148606 86.611394) (end 152.4 86.36) (width 0.25) (layer B.Cu) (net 9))
 (segment (start 170.18 88.9) (end 172.72 88.9) (width 0.25) (layer B.Cu) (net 9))
 (via (at 172.72 81.28) (size 0.6) (drill 0.4) (layers F.Cu B.Cu) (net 9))
 (segment (start 172.72 88.9) (end 172.72 81.28) (width 0.25) (layer F.Cu) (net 9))
 (via (at 172.72 88.9) (size 0.6) (drill 0.4) (layers F.Cu B.Cu) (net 9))
 (segment (start 163.466163 81.028606) (end 162.811394 81.028606) (width 0.25) (layer B.Cu) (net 9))
 (segment (start 162.811394 81.028606) (end 162.56 81.28) (width 0.25) (layer B.Cu) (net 9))
 (segment (start 163.466163 81.028606) (end 164.848606 81.028606) (width 0.25) (layer B.Cu) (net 9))
 (segment (start 164.848606 81.028606) (end 165.1 81.28) (width 0.25) (layer B.Cu) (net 9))
 (segment (start 165.1 81.28) (end 172.72 81.28) (width 0.25) (layer B.Cu) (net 9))
 (segment (start 170.18 88.9) (end 165.1 88.9) (width 0.25) (layer B.Cu) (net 9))
 (segment (start 167.64 109.22) (end 165.1 109.22) (width 0.25) (layer B.Cu) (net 9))
 (via (at 165.1 88.9) (size 0.6) (drill 0.4) (layers F.Cu B.Cu) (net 9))
 (segment (start 165.1 109.22) (end 165.1 88.9) (width 0.25) (layer F.Cu) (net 9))
 (via (at 165.1 109.22) (size 0.6) (drill 0.4) (layers F.Cu B.Cu) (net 9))
 (segment (start 157.48 83.82) (end 182.88 83.82) (width 0.25) (layer B.Cu) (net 1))
 (via (at 182.88 106.68) (size 0.6) (drill 0.4) (layers F.Cu B.Cu) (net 1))
 (segment (start 182.88 83.82) (end 182.88 106.68) (width 0.25) (layer F.Cu) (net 1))
 (via (at 182.88 83.82) (size 0.6) (drill 0.4) (layers F.Cu B.Cu) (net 1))
 (segment (start 195.58 114.3) (end 193.04 114.3) (width 0.25) (layer B.Cu) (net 1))
 (segment (start 193.04 106.68) (end 195.58 106.68) (width 0.25) (layer B.Cu) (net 1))
 (via (at 193.04 106.68) (size 0.6) (drill 0.4) (layers F.Cu B.Cu) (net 1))
 (segment (start 193.04 114.3) (end 193.04 106.68) (width 0.25) (layer F.Cu) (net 1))
 (via (at 193.04 114.3) (size 0.6) (drill 0.4) (layers F.Cu B.Cu) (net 1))
 (segment (start 195.58 106.68) (end 187.96 106.68) (width 0.25) (layer B.Cu) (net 1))
 (segment (start 187.96 106.68) (end 182.88 106.68) (width 0.25) (layer B.Cu) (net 1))
 (segment (start 182.88 106.68) (end 180.34 106.68) (width 0.25) (layer B.Cu) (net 1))
 (segment (start 180.34 106.68) (end 170.18 106.68) (width 0.25) (layer B.Cu) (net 1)))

